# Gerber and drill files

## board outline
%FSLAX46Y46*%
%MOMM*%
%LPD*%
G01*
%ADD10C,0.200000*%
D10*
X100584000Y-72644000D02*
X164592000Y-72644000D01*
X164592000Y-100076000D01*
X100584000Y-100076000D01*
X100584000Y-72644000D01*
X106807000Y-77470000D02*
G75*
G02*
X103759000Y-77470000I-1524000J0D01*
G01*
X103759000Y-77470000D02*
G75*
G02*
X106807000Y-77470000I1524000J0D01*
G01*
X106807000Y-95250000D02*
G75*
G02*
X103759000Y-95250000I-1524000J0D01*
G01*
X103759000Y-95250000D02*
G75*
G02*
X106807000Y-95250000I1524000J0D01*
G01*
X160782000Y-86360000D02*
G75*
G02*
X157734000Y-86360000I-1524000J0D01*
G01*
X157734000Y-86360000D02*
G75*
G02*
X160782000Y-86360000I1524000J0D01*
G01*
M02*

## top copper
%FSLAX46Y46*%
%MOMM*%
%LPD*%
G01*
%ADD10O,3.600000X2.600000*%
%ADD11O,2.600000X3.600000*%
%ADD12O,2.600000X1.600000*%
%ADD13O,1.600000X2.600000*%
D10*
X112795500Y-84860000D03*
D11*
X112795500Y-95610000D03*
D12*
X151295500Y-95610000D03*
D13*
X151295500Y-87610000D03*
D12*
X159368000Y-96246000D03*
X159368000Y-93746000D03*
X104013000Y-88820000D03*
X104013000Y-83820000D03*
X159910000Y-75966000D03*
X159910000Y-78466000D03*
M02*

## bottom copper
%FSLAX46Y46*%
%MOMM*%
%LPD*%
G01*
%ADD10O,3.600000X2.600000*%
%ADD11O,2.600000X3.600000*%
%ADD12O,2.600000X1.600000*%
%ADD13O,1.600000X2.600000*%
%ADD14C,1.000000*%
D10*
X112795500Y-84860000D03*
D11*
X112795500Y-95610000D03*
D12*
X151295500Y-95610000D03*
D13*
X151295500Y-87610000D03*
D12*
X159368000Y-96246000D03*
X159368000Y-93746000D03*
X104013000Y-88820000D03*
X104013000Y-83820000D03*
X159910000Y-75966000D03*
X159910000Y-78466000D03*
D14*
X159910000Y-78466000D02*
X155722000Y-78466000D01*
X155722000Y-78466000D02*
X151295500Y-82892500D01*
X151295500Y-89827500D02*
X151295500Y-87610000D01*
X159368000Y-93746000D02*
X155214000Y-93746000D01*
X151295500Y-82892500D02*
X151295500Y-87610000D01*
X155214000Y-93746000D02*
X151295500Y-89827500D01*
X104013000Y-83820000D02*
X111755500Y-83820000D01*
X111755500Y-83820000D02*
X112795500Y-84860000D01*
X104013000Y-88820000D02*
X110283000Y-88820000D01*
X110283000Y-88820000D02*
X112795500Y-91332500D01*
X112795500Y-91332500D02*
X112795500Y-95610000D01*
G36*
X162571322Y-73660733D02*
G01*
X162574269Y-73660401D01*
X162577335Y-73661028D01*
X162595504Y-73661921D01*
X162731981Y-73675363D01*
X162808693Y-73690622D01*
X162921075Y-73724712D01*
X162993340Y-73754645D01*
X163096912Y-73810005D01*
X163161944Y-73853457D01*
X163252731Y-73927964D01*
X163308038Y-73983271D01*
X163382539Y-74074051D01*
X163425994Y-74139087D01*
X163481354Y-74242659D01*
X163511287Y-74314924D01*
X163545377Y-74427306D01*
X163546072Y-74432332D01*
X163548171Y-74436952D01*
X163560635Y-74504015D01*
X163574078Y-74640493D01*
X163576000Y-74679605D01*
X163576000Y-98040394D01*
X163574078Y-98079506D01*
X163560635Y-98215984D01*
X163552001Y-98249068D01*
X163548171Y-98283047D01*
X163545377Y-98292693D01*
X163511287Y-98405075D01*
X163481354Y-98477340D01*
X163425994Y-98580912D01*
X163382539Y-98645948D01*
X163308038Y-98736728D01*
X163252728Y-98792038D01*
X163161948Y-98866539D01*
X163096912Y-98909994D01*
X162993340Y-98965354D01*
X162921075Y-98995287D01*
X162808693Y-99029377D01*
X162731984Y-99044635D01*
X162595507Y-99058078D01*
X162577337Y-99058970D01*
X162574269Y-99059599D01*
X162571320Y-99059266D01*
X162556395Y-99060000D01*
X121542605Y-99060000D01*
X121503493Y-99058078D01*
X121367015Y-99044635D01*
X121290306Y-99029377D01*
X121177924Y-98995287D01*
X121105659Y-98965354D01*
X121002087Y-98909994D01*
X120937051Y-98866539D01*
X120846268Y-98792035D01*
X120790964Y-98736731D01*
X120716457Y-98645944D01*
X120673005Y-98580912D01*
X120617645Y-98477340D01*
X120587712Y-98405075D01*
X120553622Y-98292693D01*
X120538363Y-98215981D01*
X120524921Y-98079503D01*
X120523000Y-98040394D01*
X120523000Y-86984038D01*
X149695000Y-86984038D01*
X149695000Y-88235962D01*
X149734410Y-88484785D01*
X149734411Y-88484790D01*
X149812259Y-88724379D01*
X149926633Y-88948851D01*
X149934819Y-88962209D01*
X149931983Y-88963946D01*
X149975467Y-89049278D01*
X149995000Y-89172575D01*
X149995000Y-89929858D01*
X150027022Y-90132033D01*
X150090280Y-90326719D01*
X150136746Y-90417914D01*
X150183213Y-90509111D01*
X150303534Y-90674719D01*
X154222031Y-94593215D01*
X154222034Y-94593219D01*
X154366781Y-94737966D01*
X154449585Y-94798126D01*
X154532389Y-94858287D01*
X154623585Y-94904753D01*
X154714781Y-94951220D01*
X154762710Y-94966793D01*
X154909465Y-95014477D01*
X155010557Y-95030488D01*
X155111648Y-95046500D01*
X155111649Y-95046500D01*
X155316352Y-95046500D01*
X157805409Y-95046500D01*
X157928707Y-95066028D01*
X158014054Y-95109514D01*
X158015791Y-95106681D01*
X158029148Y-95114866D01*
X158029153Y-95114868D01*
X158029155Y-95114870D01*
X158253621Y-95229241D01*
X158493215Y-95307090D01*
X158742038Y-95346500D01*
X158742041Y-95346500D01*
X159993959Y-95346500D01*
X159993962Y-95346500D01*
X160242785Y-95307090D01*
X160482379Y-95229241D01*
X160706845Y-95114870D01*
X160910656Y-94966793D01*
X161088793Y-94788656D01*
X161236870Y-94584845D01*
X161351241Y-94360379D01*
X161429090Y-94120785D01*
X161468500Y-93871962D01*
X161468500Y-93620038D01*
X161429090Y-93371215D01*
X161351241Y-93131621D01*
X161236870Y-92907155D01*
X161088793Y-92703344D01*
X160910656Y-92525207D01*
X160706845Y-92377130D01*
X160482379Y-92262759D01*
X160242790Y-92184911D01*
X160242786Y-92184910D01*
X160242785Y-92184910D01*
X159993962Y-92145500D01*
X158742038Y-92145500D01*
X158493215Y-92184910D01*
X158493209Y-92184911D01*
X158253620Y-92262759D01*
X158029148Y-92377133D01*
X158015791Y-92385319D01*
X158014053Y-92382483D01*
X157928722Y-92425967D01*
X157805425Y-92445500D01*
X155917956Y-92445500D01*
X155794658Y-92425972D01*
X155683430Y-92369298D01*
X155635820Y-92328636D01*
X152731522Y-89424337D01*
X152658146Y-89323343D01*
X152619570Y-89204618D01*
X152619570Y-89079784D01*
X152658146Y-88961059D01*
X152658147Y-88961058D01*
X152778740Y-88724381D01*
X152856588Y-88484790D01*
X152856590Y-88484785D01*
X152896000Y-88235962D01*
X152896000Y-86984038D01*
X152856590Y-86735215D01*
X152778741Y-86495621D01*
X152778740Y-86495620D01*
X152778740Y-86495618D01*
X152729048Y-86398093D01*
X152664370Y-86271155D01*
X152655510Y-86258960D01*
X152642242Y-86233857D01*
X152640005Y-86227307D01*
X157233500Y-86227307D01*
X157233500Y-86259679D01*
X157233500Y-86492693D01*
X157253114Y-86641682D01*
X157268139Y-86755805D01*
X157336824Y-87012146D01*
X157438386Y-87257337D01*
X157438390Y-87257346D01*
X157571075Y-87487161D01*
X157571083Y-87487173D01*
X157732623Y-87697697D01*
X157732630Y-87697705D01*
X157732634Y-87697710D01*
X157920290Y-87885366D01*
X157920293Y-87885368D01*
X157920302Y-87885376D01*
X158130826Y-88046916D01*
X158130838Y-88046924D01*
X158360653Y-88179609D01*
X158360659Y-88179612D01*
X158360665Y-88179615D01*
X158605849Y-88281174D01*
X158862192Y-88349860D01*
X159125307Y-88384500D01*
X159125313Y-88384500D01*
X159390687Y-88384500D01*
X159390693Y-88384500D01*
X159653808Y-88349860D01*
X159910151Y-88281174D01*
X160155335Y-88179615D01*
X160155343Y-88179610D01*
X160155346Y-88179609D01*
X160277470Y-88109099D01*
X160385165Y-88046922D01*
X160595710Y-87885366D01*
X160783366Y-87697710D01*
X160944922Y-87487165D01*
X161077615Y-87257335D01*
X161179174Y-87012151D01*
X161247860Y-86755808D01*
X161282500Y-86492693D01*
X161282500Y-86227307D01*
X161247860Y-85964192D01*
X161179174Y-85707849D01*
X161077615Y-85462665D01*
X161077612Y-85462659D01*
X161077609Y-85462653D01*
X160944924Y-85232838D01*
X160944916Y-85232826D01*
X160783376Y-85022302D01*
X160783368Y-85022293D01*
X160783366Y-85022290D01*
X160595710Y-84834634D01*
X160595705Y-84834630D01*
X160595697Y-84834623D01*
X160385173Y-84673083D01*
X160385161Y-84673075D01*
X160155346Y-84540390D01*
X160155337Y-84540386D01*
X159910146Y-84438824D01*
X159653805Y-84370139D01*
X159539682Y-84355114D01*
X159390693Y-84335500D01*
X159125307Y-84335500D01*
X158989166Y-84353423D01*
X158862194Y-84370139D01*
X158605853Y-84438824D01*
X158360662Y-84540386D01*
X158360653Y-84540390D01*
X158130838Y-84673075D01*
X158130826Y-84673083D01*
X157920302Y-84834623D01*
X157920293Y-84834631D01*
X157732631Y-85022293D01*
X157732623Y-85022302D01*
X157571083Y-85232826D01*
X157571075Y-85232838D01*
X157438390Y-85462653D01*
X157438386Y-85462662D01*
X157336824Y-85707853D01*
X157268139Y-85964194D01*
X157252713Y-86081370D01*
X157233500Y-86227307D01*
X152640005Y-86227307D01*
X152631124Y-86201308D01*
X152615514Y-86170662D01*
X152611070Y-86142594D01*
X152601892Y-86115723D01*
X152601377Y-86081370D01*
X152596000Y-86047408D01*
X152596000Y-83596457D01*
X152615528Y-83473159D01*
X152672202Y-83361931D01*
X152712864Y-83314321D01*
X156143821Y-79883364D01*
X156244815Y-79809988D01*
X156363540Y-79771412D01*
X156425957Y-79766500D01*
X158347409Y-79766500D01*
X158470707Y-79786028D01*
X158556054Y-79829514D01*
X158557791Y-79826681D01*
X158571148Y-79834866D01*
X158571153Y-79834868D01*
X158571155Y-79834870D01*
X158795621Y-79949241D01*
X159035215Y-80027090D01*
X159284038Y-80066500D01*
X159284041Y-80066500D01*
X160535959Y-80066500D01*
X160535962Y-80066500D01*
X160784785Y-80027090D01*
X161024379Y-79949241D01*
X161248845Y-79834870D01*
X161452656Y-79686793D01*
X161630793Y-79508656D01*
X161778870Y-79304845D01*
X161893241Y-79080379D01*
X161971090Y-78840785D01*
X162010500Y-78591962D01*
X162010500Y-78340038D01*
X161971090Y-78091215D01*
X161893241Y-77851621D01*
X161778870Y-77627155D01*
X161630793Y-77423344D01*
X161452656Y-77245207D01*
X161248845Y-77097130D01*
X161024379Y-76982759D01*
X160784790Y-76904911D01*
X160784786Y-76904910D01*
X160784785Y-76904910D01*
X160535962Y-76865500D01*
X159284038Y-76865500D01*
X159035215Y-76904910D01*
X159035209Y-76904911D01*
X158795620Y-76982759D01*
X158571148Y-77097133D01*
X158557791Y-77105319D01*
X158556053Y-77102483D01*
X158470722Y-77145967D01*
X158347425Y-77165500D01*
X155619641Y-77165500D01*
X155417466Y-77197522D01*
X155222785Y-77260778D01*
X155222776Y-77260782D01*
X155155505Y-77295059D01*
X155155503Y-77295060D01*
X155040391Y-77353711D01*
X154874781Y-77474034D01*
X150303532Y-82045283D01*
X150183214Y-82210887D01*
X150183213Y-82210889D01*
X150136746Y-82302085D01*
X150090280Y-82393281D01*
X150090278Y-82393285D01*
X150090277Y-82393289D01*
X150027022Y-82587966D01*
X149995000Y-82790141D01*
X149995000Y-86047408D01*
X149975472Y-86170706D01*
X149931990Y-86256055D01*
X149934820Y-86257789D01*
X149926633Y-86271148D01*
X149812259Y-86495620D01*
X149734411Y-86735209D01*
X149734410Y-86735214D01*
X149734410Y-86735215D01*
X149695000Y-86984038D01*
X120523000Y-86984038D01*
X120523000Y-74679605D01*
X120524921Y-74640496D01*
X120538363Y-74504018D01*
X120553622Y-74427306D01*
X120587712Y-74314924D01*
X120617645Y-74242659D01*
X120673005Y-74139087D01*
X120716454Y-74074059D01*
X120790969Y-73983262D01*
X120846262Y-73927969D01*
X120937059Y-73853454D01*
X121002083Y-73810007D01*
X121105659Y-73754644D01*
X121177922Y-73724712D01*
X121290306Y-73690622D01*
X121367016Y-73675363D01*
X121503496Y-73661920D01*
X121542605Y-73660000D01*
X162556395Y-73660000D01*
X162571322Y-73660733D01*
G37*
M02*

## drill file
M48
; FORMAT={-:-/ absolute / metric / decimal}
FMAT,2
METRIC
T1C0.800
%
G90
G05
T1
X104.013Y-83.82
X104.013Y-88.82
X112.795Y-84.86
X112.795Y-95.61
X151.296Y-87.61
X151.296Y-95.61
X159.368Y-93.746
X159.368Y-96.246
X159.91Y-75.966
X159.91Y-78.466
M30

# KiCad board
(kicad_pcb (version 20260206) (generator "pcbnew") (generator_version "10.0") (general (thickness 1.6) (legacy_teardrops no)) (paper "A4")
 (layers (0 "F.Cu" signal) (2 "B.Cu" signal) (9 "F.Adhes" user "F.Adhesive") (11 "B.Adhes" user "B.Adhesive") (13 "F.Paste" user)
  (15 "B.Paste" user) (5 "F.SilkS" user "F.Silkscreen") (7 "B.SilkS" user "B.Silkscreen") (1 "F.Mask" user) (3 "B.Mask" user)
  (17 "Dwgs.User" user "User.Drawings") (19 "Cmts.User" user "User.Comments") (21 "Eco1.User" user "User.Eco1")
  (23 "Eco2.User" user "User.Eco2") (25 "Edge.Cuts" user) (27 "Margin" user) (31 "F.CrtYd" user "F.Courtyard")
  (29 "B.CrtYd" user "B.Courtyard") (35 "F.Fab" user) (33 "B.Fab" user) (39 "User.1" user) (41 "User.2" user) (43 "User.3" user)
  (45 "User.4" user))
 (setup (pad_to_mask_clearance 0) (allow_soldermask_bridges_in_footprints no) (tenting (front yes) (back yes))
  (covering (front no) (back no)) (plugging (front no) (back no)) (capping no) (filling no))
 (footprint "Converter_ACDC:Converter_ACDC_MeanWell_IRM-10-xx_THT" (layer "F.Cu") (at 112.7955 84.86)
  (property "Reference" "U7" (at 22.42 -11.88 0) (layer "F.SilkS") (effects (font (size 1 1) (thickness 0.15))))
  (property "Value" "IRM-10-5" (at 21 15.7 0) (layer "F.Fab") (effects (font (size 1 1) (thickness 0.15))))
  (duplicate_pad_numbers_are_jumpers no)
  (pad "1" thru_hole oval (at 0 0) (size 3.6 2.6) (drill 0.8) (layers "*.Cu" "*.Mask") (remove_unused_layers no) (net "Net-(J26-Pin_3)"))
  (pad "2" thru_hole oval (at 0 10.75 90) (size 3.6 2.6) (drill 0.8) (layers "*.Cu" "*.Mask") (remove_unused_layers no)
   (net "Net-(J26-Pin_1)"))
  (pad "3" thru_hole oval (at 38.5 10.75) (size 2.6 1.6) (drill 0.8) (layers "*.Cu" "*.Mask") (remove_unused_layers no)
   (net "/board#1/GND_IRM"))
  (pad "4" thru_hole oval (at 38.5 2.75 90) (size 2.6 1.6) (drill 0.8) (layers "*.Cu" "*.Mask") (remove_unused_layers no)
   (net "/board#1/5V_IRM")))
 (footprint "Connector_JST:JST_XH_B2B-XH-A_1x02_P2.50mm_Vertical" (layer "F.Cu") (at 159.368 96.246 90)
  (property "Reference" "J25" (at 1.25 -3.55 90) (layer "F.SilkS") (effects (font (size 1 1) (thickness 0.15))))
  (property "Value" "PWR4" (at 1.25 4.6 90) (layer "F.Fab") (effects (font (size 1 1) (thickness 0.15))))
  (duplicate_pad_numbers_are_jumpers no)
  (pad "1" thru_hole oval (at 0 0 180) (size 2.6 1.6) (drill 0.8) (layers "*.Cu" "*.Mask") (remove_unused_layers no)
   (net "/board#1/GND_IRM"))
  (pad "2" thru_hole oval (at 2.5 0 180) (size 2.6 1.6) (drill 0.8) (layers "*.Cu" "*.Mask") (remove_unused_layers no)
   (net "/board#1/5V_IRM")))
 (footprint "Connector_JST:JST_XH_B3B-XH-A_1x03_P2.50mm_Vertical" (layer "F.Cu") (at 104.013 88.82 90)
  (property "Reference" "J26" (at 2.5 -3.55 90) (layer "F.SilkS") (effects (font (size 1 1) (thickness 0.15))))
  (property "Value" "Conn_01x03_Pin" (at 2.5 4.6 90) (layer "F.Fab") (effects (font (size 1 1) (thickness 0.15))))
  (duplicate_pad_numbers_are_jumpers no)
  (pad "1" thru_hole oval (at 0 0 180) (size 2.6 1.6) (drill 0.8) (layers "*.Cu" "*.Mask") (remove_unused_layers no) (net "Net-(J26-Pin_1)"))
  (pad "3" thru_hole oval (at 5 0 180) (size 2.6 1.6) (drill 0.8) (layers "*.Cu" "*.Mask") (remove_unused_layers no) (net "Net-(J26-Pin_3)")))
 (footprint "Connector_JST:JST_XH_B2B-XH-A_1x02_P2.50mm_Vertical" (layer "F.Cu") (at 159.91 75.966 -90)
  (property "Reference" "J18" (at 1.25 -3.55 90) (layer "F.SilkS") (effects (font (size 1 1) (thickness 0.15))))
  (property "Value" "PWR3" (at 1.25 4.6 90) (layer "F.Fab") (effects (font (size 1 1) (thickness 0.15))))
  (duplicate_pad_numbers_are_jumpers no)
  (pad "1" thru_hole oval (at 0 0) (size 2.6 1.6) (drill 0.8) (layers "*.Cu" "*.Mask") (remove_unused_layers no) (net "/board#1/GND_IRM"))
  (pad "2" thru_hole oval (at 2.5 0) (size 2.6 1.6) (drill 0.8) (layers "*.Cu" "*.Mask") (remove_unused_layers no) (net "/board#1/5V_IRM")))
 (gr_rect (start 100.584 72.644) (end 164.592 100.076) (stroke (width 0.2) (type solid)) (fill no) (layer "Edge.Cuts"))
 (gr_circle (center 105.283 77.47) (end 106.807 77.47) (stroke (width 0.2) (type solid)) (fill no) (layer "Edge.Cuts"))
 (gr_circle (center 105.283 95.25) (end 106.807 95.25) (stroke (width 0.2) (type solid)) (fill no) (layer "Edge.Cuts"))
 (gr_circle (center 159.258 86.36) (end 160.782 86.36) (stroke (width 0.2) (type solid)) (fill no) (layer "Edge.Cuts"))
 (segment (start 159.91 78.466) (end 155.722 78.466) (width 1) (layer "B.Cu") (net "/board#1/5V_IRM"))
 (segment (start 155.722 78.466) (end 151.2955 82.8925) (width 1) (layer "B.Cu") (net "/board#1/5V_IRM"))
 (segment (start 151.2955 89.8275) (end 151.2955 87.61) (width 1) (layer "B.Cu") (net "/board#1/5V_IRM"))
 (segment (start 159.368 93.746) (end 155.214 93.746) (width 1) (layer "B.Cu") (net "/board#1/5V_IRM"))
 (segment (start 151.2955 82.8925) (end 151.2955 87.61) (width 1) (layer "B.Cu") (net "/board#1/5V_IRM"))
 (segment (start 155.214 93.746) (end 151.2955 89.8275) (width 1) (layer "B.Cu") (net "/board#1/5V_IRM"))
 (segment (start 104.013 83.82) (end 111.7555 83.82) (width 1) (layer "B.Cu") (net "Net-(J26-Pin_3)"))
 (segment (start 111.7555 83.82) (end 112.7955 84.86) (width 1) (layer "B.Cu") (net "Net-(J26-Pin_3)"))
 (segment (start 104.013 88.82) (end 110.283 88.82) (width 1) (layer "B.Cu") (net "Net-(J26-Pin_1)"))
 (segment (start 110.283 88.82) (end 112.7955 91.3325) (width 1) (layer "B.Cu") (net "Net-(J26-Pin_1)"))
 (segment (start 112.7955 91.3325) (end 112.7955 95.61) (width 1) (layer "B.Cu") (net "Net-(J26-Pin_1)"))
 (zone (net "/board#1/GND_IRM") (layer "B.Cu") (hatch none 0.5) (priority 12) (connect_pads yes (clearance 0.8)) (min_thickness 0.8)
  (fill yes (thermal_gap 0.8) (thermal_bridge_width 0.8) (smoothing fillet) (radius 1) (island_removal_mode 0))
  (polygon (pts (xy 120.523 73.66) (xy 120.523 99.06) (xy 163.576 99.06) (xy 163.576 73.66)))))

